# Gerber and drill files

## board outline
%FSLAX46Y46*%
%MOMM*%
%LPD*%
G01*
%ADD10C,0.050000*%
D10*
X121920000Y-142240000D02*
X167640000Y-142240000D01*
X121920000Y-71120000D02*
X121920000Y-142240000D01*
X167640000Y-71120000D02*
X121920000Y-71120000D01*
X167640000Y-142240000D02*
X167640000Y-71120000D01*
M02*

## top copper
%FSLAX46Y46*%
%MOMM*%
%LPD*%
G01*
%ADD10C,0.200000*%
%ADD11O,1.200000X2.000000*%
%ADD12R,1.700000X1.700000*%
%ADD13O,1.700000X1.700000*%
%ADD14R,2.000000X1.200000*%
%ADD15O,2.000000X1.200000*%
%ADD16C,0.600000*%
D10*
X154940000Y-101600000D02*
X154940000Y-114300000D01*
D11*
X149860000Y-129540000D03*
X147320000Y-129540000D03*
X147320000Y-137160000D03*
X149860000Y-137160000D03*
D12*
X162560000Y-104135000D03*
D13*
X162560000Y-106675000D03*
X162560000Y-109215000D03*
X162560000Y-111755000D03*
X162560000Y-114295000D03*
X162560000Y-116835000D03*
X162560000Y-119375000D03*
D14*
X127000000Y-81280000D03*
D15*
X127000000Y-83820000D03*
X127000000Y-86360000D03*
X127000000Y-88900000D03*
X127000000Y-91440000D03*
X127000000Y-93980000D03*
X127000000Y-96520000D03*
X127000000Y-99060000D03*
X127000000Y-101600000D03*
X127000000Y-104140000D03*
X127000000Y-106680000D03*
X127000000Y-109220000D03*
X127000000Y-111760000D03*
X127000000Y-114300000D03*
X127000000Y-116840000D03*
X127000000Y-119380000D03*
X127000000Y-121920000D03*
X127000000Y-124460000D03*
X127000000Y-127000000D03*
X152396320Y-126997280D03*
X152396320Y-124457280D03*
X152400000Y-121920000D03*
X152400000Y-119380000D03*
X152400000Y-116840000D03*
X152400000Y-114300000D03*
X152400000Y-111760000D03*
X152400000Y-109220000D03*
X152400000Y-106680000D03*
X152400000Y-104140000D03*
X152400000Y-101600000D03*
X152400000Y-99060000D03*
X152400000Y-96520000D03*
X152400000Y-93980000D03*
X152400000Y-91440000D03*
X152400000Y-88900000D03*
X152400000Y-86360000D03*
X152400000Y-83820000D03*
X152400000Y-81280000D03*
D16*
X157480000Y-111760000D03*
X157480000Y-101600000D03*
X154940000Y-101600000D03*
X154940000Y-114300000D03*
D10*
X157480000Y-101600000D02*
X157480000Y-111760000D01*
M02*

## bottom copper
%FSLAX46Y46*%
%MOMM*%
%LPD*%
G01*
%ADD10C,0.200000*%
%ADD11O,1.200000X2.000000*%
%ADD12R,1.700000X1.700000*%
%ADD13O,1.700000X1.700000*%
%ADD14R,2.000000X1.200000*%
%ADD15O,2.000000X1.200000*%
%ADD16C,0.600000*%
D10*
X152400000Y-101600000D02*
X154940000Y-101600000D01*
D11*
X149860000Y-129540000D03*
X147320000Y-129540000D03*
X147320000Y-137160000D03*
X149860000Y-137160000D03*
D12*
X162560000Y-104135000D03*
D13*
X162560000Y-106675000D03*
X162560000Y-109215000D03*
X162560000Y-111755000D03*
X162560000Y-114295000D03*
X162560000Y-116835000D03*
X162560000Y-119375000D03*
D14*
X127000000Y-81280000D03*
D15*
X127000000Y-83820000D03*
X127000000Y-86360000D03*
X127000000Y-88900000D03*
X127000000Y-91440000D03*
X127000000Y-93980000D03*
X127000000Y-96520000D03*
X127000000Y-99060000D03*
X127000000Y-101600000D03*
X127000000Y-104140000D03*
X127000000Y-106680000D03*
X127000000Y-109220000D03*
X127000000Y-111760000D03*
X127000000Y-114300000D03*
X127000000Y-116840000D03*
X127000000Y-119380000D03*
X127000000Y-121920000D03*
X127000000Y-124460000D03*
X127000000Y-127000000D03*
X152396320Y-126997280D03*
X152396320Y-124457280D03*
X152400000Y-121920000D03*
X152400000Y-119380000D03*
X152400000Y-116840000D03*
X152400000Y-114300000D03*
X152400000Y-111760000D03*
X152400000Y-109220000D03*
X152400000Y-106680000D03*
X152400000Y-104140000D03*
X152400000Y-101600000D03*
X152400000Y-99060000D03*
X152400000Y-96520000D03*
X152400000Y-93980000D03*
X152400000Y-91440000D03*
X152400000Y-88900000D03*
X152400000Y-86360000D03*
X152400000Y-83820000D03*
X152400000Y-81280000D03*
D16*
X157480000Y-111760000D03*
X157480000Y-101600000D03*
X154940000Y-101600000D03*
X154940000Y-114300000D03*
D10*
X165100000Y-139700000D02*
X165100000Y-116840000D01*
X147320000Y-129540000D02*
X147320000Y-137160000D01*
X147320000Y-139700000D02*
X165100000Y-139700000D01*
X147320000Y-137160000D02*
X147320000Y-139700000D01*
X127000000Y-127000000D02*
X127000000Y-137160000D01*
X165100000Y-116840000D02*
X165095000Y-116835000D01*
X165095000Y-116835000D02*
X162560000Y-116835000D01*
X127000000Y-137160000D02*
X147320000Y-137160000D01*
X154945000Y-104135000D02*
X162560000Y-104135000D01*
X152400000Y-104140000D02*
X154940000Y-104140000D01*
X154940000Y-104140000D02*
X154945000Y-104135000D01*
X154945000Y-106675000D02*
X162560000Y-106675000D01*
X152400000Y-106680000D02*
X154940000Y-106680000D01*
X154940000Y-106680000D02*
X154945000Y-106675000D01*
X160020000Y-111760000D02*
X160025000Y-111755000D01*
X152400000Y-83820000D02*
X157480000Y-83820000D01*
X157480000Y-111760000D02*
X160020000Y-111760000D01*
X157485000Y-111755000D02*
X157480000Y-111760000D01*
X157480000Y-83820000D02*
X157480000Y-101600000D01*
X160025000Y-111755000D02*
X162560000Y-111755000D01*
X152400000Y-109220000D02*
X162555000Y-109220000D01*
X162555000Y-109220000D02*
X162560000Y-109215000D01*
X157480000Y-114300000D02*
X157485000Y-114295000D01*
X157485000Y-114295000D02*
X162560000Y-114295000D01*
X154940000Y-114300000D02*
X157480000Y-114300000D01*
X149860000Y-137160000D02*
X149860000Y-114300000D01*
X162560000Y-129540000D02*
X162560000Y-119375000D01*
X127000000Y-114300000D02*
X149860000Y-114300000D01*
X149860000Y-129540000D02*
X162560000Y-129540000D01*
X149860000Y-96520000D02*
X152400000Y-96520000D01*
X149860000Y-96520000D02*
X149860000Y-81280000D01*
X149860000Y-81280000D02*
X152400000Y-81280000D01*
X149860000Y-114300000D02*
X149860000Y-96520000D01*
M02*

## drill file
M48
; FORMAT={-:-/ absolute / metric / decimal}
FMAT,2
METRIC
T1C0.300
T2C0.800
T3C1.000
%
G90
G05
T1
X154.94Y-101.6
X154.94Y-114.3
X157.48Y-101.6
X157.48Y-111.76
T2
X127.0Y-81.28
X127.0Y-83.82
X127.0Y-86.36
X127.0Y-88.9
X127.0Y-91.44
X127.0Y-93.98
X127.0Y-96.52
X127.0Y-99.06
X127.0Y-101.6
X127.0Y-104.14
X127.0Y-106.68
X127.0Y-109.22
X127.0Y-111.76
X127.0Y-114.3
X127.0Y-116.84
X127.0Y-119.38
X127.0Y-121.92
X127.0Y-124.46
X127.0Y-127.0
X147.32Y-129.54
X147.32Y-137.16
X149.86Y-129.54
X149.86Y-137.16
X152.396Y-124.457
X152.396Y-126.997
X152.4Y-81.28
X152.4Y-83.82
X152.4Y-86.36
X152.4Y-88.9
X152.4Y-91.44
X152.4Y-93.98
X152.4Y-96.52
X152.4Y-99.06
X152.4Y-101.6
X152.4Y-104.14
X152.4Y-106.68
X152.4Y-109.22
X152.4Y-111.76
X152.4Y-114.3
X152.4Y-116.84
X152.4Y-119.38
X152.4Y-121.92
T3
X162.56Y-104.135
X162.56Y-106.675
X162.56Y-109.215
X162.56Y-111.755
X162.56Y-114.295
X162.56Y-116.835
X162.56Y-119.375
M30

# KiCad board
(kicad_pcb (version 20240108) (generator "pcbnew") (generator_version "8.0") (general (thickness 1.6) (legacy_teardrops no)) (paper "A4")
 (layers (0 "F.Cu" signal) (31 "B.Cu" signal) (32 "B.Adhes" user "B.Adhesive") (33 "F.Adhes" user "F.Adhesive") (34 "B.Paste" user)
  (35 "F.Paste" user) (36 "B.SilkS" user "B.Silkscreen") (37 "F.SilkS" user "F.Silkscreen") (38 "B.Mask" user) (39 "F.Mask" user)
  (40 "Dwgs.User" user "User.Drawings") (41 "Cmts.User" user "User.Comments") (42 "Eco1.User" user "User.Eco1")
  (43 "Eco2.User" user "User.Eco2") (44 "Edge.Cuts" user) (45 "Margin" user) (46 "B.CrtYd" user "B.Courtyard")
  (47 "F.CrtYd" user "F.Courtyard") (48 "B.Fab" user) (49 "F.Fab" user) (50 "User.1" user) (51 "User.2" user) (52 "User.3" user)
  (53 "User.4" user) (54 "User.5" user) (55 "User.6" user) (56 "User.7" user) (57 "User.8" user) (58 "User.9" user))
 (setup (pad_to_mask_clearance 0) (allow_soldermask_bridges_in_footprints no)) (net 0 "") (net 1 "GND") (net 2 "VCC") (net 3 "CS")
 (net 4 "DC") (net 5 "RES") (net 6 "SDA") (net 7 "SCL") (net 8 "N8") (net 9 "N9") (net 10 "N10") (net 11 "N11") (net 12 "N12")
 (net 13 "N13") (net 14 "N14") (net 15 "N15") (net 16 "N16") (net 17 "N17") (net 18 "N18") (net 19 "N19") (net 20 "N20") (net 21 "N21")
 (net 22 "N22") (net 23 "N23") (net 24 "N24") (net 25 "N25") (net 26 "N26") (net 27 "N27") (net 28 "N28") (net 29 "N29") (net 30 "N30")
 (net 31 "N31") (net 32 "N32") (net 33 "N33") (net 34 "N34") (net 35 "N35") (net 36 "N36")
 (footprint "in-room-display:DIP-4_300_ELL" (layer "F.Cu") (at 148.59 133.35 180)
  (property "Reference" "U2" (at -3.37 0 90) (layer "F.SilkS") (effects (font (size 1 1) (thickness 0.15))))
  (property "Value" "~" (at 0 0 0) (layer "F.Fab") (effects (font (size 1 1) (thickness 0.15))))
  (pad "1" thru_hole oval (at -1.27 3.81 180) (size 1.2 2) (drill 0.8) (layers "*.Cu" "*.Mask") (remove_unused_layers no) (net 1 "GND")
   (thermal_bridge_angle 45))
  (pad "2" thru_hole oval (at 1.27 3.81 180) (size 1.2 2) (drill 0.8) (layers "*.Cu" "*.Mask") (remove_unused_layers no) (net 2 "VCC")
   (thermal_bridge_angle 45))
  (pad "3" thru_hole oval (at 1.27 -3.81 180) (size 1.2 2) (drill 0.8) (layers "*.Cu" "*.Mask") (remove_unused_layers no) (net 2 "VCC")
   (thermal_bridge_angle 45))
  (pad "4" thru_hole oval (at -1.27 -3.81 180) (size 1.2 2) (drill 0.8) (layers "*.Cu" "*.Mask") (remove_unused_layers no) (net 1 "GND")
   (thermal_bridge_angle 45)))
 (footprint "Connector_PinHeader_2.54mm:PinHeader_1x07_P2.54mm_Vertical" (layer "F.Cu") (at 162.56 104.135)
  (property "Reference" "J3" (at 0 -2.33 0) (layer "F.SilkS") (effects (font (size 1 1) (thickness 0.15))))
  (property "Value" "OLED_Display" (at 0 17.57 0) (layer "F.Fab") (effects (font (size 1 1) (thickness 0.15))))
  (pad "1" thru_hole rect (at 0 0) (size 1.7 1.7) (drill 1) (layers "*.Cu" "*.Mask") (remove_unused_layers no) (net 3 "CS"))
  (pad "2" thru_hole oval (at 0 2.54) (size 1.7 1.7) (drill 1) (layers "*.Cu" "*.Mask") (remove_unused_layers no) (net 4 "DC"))
  (pad "3" thru_hole oval (at 0 5.08) (size 1.7 1.7) (drill 1) (layers "*.Cu" "*.Mask") (remove_unused_layers no) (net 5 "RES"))
  (pad "4" thru_hole oval (at 0 7.62) (size 1.7 1.7) (drill 1) (layers "*.Cu" "*.Mask") (remove_unused_layers no) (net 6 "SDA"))
  (pad "5" thru_hole oval (at 0 10.16) (size 1.7 1.7) (drill 1) (layers "*.Cu" "*.Mask") (remove_unused_layers no) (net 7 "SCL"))
  (pad "6" thru_hole oval (at 0 12.7) (size 1.7 1.7) (drill 1) (layers "*.Cu" "*.Mask") (remove_unused_layers no) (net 2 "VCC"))
  (pad "7" thru_hole oval (at 0 15.24) (size 1.7 1.7) (drill 1) (layers "*.Cu" "*.Mask") (remove_unused_layers no) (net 1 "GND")))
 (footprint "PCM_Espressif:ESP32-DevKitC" (layer "F.Cu") (at 127 81.28)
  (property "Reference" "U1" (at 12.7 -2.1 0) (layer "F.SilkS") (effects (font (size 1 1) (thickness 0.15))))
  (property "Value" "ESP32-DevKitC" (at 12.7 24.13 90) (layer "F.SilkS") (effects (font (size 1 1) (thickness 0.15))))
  (pad "1" thru_hole rect (at 0 0 270) (size 1.2 2) (drill 0.8) (layers "*.Cu" "*.Mask") (remove_unused_layers no) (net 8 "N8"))
  (pad "2" thru_hole oval (at 0 2.54 270) (size 1.2 2) (drill 0.8) (layers "*.Cu" "*.Mask") (remove_unused_layers no) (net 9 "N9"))
  (pad "3" thru_hole oval (at 0 5.08 270) (size 1.2 2) (drill 0.8) (layers "*.Cu" "*.Mask") (remove_unused_layers no) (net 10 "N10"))
  (pad "4" thru_hole oval (at 0 7.62 270) (size 1.2 2) (drill 0.8) (layers "*.Cu" "*.Mask") (remove_unused_layers no) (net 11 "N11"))
  (pad "5" thru_hole oval (at 0 10.16 270) (size 1.2 2) (drill 0.8) (layers "*.Cu" "*.Mask") (remove_unused_layers no) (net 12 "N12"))
  (pad "6" thru_hole oval (at 0 12.7 270) (size 1.2 2) (drill 0.8) (layers "*.Cu" "*.Mask") (remove_unused_layers no) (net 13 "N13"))
  (pad "7" thru_hole oval (at 0 15.24 270) (size 1.2 2) (drill 0.8) (layers "*.Cu" "*.Mask") (remove_unused_layers no) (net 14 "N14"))
  (pad "8" thru_hole oval (at 0 17.78 270) (size 1.2 2) (drill 0.8) (layers "*.Cu" "*.Mask") (remove_unused_layers no) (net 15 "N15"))
  (pad "9" thru_hole oval (at 0 20.32 270) (size 1.2 2) (drill 0.8) (layers "*.Cu" "*.Mask") (remove_unused_layers no) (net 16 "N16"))
  (pad "10" thru_hole oval (at 0 22.86 270) (size 1.2 2) (drill 0.8) (layers "*.Cu" "*.Mask") (remove_unused_layers no) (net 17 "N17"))
  (pad "11" thru_hole oval (at 0 25.4 270) (size 1.2 2) (drill 0.8) (layers "*.Cu" "*.Mask") (remove_unused_layers no) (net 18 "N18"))
  (pad "12" thru_hole oval (at 0 27.94 270) (size 1.2 2) (drill 0.8) (layers "*.Cu" "*.Mask") (remove_unused_layers no) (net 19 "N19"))
  (pad "13" thru_hole oval (at 0 30.48 270) (size 1.2 2) (drill 0.8) (layers "*.Cu" "*.Mask") (remove_unused_layers no) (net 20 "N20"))
  (pad "14" thru_hole oval (at 0 33.02 270) (size 1.2 2) (drill 0.8) (layers "*.Cu" "*.Mask") (remove_unused_layers no) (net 1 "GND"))
  (pad "15" thru_hole oval (at 0 35.56 270) (size 1.2 2) (drill 0.8) (layers "*.Cu" "*.Mask") (remove_unused_layers no) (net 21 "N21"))
  (pad "16" thru_hole oval (at 0 38.1 270) (size 1.2 2) (drill 0.8) (layers "*.Cu" "*.Mask") (remove_unused_layers no) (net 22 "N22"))
  (pad "17" thru_hole oval (at 0 40.64 270) (size 1.2 2) (drill 0.8) (layers "*.Cu" "*.Mask") (remove_unused_layers no) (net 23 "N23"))
  (pad "18" thru_hole oval (at 0 43.18 270) (size 1.2 2) (drill 0.8) (layers "*.Cu" "*.Mask") (remove_unused_layers no) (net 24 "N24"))
  (pad "19" thru_hole oval (at 0 45.72 270) (size 1.2 2) (drill 0.8) (layers "*.Cu" "*.Mask") (remove_unused_layers no) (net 2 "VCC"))
  (pad "20" thru_hole oval (at 25.39632 45.71728 270) (size 1.2 2) (drill 0.8) (layers "*.Cu" "*.Mask") (remove_unused_layers no)
   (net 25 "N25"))
  (pad "21" thru_hole oval (at 25.39632 43.17728 270) (size 1.2 2) (drill 0.8) (layers "*.Cu" "*.Mask") (remove_unused_layers no)
   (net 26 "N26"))
  (pad "22" thru_hole oval (at 25.4 40.64 270) (size 1.2 2) (drill 0.8) (layers "*.Cu" "*.Mask") (remove_unused_layers no) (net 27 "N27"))
  (pad "23" thru_hole oval (at 25.4 38.1 270) (size 1.2 2) (drill 0.8) (layers "*.Cu" "*.Mask") (remove_unused_layers no) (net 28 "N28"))
  (pad "24" thru_hole oval (at 25.4 35.56 270) (size 1.2 2) (drill 0.8) (layers "*.Cu" "*.Mask") (remove_unused_layers no) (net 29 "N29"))
  (pad "25" thru_hole oval (at 25.4 33.02 270) (size 1.2 2) (drill 0.8) (layers "*.Cu" "*.Mask") (remove_unused_layers no) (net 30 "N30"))
  (pad "26" thru_hole oval (at 25.4 30.48 270) (size 1.2 2) (drill 0.8) (layers "*.Cu" "*.Mask") (remove_unused_layers no) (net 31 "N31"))
  (pad "27" thru_hole oval (at 25.4 27.94 270) (size 1.2 2) (drill 0.8) (layers "*.Cu" "*.Mask") (remove_unused_layers no) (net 5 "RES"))
  (pad "28" thru_hole oval (at 25.4 25.4 270) (size 1.2 2) (drill 0.8) (layers "*.Cu" "*.Mask") (remove_unused_layers no) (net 4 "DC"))
  (pad "29" thru_hole oval (at 25.4 22.86 270) (size 1.2 2) (drill 0.8) (layers "*.Cu" "*.Mask") (remove_unused_layers no) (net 3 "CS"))
  (pad "30" thru_hole oval (at 25.4 20.32 270) (size 1.2 2) (drill 0.8) (layers "*.Cu" "*.Mask") (remove_unused_layers no) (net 7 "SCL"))
  (pad "31" thru_hole oval (at 25.4 17.78 270) (size 1.2 2) (drill 0.8) (layers "*.Cu" "*.Mask") (remove_unused_layers no) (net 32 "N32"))
  (pad "32" thru_hole oval (at 25.4 15.24 270) (size 1.2 2) (drill 0.8) (layers "*.Cu" "*.Mask") (remove_unused_layers no) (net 1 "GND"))
  (pad "33" thru_hole oval (at 25.4 12.7 270) (size 1.2 2) (drill 0.8) (layers "*.Cu" "*.Mask") (remove_unused_layers no) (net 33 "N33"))
  (pad "34" thru_hole oval (at 25.4 10.16 270) (size 1.2 2) (drill 0.8) (layers "*.Cu" "*.Mask") (remove_unused_layers no) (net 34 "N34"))
  (pad "35" thru_hole oval (at 25.4 7.62 270) (size 1.2 2) (drill 0.8) (layers "*.Cu" "*.Mask") (remove_unused_layers no) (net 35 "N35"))
  (pad "36" thru_hole oval (at 25.4 5.08 270) (size 1.2 2) (drill 0.8) (layers "*.Cu" "*.Mask") (remove_unused_layers no) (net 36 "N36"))
  (pad "37" thru_hole oval (at 25.4 2.54 270) (size 1.2 2) (drill 0.8) (layers "*.Cu" "*.Mask") (remove_unused_layers no) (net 6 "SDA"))
  (pad "38" thru_hole oval (at 25.4 0 270) (size 1.2 2) (drill 0.8) (layers "*.Cu" "*.Mask") (remove_unused_layers no) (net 1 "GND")))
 (gr_line (start 154.94 101.6) (end 154.94 114.3) (stroke (width 0.2) (type default)) (layer "F.Cu") (net 7))
 (gr_line (start 152.4 101.6) (end 154.94 101.6) (stroke (width 0.2) (type default)) (layer "B.Cu") (net 7))
 (gr_line (start 121.92 142.24) (end 167.64 142.24) (stroke (width 0.05) (type default)) (layer "Edge.Cuts"))
 (gr_line (start 121.92 71.12) (end 121.92 142.24) (stroke (width 0.05) (type default)) (layer "Edge.Cuts"))
 (gr_line (start 167.64 71.12) (end 121.92 71.12) (stroke (width 0.05) (type default)) (layer "Edge.Cuts"))
 (gr_line (start 167.64 142.24) (end 167.64 71.12) (stroke (width 0.05) (type default)) (layer "Edge.Cuts"))
 (segment (start 165.1 139.7) (end 165.1 116.84) (width 0.2) (layer "B.Cu") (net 2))
 (segment (start 147.32 129.54) (end 147.32 137.16) (width 0.2) (layer "B.Cu") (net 2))
 (segment (start 147.32 139.7) (end 165.1 139.7) (width 0.2) (layer "B.Cu") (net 2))
 (segment (start 147.32 137.16) (end 147.32 139.7) (width 0.2) (layer "B.Cu") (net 2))
 (segment (start 127 127) (end 127 137.16) (width 0.2) (layer "B.Cu") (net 2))
 (segment (start 165.1 116.84) (end 165.095 116.835) (width 0.2) (layer "B.Cu") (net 2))
 (segment (start 165.095 116.835) (end 162.56 116.835) (width 0.2) (layer "B.Cu") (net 2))
 (segment (start 127 137.16) (end 147.32 137.16) (width 0.2) (layer "B.Cu") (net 2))
 (segment (start 154.945 104.135) (end 162.56 104.135) (width 0.2) (layer "B.Cu") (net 3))
 (segment (start 152.4 104.14) (end 154.94 104.14) (width 0.2) (layer "B.Cu") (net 3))
 (segment (start 154.94 104.14) (end 154.945 104.135) (width 0.2) (layer "B.Cu") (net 3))
 (segment (start 154.945 106.675) (end 162.56 106.675) (width 0.2) (layer "B.Cu") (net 4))
 (segment (start 152.4 106.68) (end 154.94 106.68) (width 0.2) (layer "B.Cu") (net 4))
 (segment (start 154.94 106.68) (end 154.945 106.675) (width 0.2) (layer "B.Cu") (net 4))
 (segment (start 157.48 101.6) (end 157.48 111.76) (width 0.2) (layer "F.Cu") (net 6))
 (via (at 157.48 111.76) (size 0.6) (drill 0.3) (layers "F.Cu" "B.Cu") (free yes) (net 6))
 (via (at 157.48 101.6) (size 0.6) (drill 0.3) (layers "F.Cu" "B.Cu") (free yes) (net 6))
 (segment (start 160.02 111.76) (end 160.025 111.755) (width 0.2) (layer "B.Cu") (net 6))
 (segment (start 152.4 83.82) (end 157.48 83.82) (width 0.2) (layer "B.Cu") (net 6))
 (segment (start 157.48 111.76) (end 160.02 111.76) (width 0.2) (layer "B.Cu") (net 6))
 (segment (start 157.485 111.755) (end 157.48 111.76) (width 0.2) (layer "B.Cu") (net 6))
 (segment (start 157.48 83.82) (end 157.48 101.6) (width 0.2) (layer "B.Cu") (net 6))
 (segment (start 160.025 111.755) (end 162.56 111.755) (width 0.2) (layer "B.Cu") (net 6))
 (segment (start 152.4 109.22) (end 162.555 109.22) (width 0.2) (layer "B.Cu") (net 5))
 (segment (start 162.555 109.22) (end 162.56 109.215) (width 0.2) (layer "B.Cu") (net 5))
 (via (at 154.94 101.6) (size 0.6) (drill 0.3) (layers "F.Cu" "B.Cu") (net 7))
 (via (at 154.94 114.3) (size 0.6) (drill 0.3) (layers "F.Cu" "B.Cu") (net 7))
 (segment (start 157.48 114.3) (end 157.485 114.295) (width 0.2) (layer "B.Cu") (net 7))
 (segment (start 157.485 114.295) (end 162.56 114.295) (width 0.2) (layer "B.Cu") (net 7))
 (segment (start 154.94 114.3) (end 157.48 114.3) (width 0.2) (layer "B.Cu") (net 7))
 (segment (start 149.86 137.16) (end 149.86 114.3) (width 0.2) (layer "B.Cu") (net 1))
 (segment (start 162.56 129.54) (end 162.56 119.375) (width 0.2) (layer "B.Cu") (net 1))
 (segment (start 127 114.3) (end 149.86 114.3) (width 0.2) (layer "B.Cu") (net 1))
 (segment (start 149.86 129.54) (end 162.56 129.54) (width 0.2) (layer "B.Cu") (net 1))
 (segment (start 149.86 96.52) (end 152.4 96.52) (width 0.2) (layer "B.Cu") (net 1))
 (segment (start 149.86 96.52) (end 149.86 81.28) (width 0.2) (layer "B.Cu") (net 1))
 (segment (start 149.86 81.28) (end 152.4 81.28) (width 0.2) (layer "B.Cu") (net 1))
 (segment (start 149.86 114.3) (end 149.86 96.52) (width 0.2) (layer "B.Cu") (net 1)))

